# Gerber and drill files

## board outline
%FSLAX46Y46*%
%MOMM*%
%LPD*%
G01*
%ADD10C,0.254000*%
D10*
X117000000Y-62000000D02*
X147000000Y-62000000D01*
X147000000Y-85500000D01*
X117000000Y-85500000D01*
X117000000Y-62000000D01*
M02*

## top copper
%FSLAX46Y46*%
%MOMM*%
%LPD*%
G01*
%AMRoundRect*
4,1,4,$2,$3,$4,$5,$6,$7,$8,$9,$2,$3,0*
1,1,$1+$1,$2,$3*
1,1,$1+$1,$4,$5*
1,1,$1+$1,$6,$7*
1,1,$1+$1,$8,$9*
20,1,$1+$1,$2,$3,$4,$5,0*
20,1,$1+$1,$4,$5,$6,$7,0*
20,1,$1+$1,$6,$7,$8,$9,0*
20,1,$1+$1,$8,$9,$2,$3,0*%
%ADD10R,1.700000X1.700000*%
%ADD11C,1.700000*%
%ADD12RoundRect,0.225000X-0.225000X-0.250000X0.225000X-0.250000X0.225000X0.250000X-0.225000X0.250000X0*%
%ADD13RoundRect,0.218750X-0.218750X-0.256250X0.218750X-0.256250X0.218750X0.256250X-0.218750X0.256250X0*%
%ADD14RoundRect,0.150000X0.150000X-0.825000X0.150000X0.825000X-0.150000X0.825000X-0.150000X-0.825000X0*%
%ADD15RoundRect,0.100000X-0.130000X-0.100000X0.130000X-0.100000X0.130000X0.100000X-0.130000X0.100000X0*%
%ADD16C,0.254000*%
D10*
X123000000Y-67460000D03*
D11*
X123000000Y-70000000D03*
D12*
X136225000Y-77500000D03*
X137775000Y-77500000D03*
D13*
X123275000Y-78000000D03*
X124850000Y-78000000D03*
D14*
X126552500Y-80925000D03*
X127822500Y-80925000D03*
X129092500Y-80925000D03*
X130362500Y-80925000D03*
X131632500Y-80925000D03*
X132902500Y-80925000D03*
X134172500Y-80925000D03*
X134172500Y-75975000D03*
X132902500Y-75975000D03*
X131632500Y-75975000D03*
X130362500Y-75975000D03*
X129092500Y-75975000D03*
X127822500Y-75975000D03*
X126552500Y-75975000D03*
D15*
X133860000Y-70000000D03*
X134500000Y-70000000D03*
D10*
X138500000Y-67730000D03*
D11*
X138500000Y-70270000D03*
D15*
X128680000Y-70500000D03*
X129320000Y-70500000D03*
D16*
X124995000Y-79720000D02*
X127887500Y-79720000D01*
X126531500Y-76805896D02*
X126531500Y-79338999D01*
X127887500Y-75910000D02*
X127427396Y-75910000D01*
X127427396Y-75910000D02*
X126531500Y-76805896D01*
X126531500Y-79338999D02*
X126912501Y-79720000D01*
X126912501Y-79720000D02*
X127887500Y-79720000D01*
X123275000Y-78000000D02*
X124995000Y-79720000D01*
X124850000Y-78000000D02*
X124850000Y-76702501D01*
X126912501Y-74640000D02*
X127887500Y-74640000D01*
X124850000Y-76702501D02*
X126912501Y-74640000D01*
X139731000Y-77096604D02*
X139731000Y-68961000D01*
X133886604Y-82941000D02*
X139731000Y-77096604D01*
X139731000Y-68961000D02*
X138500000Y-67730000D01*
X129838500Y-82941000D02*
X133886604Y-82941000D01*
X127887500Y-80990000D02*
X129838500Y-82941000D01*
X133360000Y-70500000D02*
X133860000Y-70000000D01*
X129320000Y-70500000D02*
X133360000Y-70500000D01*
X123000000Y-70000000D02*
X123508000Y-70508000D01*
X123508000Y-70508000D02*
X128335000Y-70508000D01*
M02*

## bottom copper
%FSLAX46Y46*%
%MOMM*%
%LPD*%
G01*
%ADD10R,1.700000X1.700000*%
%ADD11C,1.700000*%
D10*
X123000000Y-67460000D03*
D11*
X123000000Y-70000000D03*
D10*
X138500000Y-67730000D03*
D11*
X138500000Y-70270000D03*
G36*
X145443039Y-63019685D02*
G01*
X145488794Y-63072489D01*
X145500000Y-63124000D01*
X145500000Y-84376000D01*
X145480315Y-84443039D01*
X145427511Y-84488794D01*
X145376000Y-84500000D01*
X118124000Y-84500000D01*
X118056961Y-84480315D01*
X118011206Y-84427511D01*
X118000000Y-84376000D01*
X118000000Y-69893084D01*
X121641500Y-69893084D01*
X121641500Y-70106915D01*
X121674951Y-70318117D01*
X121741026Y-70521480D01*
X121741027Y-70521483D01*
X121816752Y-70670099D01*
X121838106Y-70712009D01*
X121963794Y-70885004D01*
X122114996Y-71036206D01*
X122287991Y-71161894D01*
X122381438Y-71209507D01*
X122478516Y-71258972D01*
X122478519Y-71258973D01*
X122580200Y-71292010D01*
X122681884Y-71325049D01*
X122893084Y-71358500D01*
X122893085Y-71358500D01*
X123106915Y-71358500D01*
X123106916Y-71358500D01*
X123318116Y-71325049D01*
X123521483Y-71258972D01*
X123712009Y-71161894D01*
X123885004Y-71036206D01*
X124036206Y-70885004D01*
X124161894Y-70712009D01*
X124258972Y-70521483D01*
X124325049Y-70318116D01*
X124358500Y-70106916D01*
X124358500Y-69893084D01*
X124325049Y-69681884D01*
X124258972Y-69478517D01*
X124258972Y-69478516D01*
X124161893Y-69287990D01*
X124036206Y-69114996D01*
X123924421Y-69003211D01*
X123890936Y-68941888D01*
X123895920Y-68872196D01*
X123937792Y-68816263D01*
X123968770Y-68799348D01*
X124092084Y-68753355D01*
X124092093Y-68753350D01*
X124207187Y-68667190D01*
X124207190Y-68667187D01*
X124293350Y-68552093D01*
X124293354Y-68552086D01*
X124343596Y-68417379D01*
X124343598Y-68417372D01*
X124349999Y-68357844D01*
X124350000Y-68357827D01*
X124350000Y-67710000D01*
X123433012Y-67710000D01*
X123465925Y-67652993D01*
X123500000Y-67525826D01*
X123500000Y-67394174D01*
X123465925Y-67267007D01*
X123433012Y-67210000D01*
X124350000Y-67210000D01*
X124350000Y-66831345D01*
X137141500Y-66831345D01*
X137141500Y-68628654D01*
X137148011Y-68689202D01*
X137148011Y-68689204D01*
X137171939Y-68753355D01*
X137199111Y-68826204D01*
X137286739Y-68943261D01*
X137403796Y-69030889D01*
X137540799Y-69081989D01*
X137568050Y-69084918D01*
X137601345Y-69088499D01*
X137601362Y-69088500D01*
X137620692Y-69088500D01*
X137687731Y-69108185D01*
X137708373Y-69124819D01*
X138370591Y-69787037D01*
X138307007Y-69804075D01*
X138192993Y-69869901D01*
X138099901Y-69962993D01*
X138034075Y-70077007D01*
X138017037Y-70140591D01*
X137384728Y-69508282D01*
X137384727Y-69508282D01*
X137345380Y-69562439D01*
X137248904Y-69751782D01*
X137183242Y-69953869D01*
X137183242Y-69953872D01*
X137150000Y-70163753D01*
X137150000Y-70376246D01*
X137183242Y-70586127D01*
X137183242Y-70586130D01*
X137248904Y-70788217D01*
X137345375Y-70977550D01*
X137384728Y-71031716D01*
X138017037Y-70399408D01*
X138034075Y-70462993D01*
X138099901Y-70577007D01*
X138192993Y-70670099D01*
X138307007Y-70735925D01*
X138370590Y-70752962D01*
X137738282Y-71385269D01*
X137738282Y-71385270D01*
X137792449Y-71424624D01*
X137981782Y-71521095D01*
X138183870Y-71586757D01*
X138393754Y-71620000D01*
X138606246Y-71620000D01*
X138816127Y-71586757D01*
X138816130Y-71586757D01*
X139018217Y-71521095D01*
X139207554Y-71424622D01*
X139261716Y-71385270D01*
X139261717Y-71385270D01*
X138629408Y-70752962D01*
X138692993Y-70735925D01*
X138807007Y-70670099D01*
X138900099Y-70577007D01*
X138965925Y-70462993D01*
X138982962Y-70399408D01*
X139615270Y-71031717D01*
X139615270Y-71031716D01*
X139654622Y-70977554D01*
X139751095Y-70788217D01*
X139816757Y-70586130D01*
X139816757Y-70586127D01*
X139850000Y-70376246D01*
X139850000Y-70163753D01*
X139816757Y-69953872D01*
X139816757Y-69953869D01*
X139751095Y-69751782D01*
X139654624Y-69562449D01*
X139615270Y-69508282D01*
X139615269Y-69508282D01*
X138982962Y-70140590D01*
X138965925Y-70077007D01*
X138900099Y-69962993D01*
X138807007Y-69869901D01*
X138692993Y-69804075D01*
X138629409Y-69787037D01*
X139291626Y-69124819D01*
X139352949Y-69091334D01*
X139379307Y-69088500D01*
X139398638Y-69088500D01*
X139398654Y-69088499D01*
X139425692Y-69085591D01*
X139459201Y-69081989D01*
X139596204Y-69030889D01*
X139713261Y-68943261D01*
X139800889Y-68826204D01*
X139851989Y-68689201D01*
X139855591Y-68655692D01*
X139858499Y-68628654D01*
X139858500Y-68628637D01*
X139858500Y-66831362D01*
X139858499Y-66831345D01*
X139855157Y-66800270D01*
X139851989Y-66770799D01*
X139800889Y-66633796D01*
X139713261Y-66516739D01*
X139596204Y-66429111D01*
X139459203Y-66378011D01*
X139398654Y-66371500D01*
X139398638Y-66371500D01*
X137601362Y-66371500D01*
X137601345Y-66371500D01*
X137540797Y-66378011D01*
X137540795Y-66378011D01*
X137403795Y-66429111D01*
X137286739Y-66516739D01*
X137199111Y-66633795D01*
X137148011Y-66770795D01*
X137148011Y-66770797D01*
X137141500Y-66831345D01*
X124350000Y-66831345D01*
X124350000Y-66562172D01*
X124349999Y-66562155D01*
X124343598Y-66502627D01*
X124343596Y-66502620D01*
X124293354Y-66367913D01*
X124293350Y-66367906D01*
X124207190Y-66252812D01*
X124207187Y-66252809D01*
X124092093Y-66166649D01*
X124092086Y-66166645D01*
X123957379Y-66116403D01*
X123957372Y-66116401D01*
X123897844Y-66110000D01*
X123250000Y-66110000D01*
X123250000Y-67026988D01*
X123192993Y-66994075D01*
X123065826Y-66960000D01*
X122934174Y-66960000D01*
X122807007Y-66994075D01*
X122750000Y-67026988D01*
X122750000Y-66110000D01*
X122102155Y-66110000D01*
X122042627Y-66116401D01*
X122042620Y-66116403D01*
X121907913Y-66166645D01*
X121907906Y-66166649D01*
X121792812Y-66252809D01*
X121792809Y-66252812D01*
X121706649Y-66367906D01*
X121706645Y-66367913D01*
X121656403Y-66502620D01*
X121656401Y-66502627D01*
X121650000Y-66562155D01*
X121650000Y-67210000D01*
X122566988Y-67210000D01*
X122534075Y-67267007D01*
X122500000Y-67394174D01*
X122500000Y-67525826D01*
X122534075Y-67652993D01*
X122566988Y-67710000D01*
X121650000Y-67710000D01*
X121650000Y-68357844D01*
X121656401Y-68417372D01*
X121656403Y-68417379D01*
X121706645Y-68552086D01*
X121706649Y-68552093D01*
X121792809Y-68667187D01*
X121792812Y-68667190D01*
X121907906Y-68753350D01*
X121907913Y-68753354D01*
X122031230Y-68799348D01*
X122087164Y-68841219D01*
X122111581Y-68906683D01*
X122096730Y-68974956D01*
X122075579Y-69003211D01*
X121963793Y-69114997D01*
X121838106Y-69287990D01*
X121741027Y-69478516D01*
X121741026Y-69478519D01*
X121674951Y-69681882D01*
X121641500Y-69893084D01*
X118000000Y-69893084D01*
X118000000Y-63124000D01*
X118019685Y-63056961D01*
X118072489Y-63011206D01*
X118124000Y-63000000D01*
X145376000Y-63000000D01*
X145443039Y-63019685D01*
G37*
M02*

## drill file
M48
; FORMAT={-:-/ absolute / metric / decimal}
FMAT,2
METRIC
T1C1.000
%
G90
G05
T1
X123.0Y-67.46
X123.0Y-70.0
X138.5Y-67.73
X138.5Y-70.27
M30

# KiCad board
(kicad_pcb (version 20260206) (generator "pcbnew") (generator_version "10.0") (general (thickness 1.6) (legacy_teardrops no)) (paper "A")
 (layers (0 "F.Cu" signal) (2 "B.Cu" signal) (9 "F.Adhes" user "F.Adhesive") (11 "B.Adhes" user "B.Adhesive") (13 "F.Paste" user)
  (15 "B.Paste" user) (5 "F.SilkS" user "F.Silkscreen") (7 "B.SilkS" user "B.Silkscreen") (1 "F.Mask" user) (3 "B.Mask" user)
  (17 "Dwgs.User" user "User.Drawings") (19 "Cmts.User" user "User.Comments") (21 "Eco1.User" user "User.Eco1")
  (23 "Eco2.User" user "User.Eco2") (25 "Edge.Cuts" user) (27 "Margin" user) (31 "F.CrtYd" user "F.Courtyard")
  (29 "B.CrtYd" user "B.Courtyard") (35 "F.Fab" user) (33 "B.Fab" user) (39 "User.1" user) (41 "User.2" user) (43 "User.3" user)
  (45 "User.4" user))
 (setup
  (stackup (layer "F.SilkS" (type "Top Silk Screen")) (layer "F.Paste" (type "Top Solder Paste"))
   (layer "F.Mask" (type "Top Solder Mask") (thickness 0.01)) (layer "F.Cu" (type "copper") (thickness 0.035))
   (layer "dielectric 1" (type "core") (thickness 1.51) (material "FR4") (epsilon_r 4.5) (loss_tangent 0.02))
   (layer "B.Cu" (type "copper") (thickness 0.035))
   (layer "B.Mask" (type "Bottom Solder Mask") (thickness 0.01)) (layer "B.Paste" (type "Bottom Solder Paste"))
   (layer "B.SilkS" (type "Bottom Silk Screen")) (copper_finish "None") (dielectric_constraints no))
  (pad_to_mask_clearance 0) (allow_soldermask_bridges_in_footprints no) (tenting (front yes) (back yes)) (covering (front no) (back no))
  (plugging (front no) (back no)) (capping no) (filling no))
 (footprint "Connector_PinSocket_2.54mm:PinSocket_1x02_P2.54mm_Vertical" (layer "F.Cu") (at 123 67.46)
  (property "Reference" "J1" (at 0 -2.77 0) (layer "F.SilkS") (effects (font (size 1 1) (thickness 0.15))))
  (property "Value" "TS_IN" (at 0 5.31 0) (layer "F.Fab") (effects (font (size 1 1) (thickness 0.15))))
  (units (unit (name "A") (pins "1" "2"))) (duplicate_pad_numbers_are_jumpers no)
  (pad "1" thru_hole rect (at 0 0) (size 1.7 1.7) (drill 1) (layers "*.Cu" "*.Mask") (remove_unused_layers no) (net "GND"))
  (pad "2" thru_hole circle (at 0 2.54) (size 1.7 1.7) (drill 1) (layers "*.Cu" "*.Mask") (remove_unused_layers no) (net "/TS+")))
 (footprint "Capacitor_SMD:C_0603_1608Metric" (layer "F.Cu") (at 137 77.5)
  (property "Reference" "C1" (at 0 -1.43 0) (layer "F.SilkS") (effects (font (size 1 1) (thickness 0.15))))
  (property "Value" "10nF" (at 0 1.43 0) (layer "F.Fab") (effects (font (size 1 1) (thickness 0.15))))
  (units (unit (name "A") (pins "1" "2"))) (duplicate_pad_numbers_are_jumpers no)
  (pad "1" smd roundrect (at -0.775 0) (size 0.9 0.95) (layers "F.Cu" "F.Mask" "F.Paste") (roundrect_rratio 0.25) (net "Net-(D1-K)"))
  (pad "2" smd roundrect (at 0.775 0) (size 0.9 0.95) (layers "F.Cu" "F.Mask" "F.Paste") (roundrect_rratio 0.25) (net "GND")))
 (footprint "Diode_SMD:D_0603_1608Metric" (layer "F.Cu") (at 124.0625 78)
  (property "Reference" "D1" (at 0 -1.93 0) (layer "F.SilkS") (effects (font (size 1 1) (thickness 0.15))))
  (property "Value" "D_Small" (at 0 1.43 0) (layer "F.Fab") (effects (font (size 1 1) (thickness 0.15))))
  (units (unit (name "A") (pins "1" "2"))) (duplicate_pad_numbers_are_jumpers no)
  (pad "1" smd roundrect (at -0.7875 0) (size 0.875 0.95) (layers "F.Cu" "F.Mask" "F.Paste") (roundrect_rratio 0.25) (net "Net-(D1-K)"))
  (pad "2" smd roundrect (at 0.7875 0) (size 0.875 0.95) (layers "F.Cu" "F.Mask" "F.Paste") (roundrect_rratio 0.25) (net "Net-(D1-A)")))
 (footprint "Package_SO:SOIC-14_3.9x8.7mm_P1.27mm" (layer "F.Cu") (at 130.3625 78.45 90)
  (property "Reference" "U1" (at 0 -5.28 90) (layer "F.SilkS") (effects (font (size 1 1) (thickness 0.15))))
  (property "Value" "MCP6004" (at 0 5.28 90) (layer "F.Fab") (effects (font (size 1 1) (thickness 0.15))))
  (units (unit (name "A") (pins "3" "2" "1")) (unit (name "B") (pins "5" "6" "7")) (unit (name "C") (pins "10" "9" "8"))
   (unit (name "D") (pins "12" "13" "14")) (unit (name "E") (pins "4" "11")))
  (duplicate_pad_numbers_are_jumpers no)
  (pad "1" smd roundrect (at -2.475 -3.81 90) (size 1.95 0.6) (layers "F.Cu" "F.Mask" "F.Paste") (roundrect_rratio 0.25) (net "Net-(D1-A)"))
  (pad "2" smd roundrect (at -2.475 -2.54 90) (size 1.95 0.6) (layers "F.Cu" "F.Mask" "F.Paste") (roundrect_rratio 0.25) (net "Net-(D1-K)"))
  (pad "3" smd roundrect (at -2.475 -1.27 90) (size 1.95 0.6) (layers "F.Cu" "F.Mask" "F.Paste") (roundrect_rratio 0.25) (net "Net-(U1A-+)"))
  (pad "4" smd roundrect (at -2.475 0 90) (size 1.95 0.6) (layers "F.Cu" "F.Mask" "F.Paste") (roundrect_rratio 0.25))
  (pad "5" smd roundrect (at -2.475 1.27 90) (size 1.95 0.6) (layers "F.Cu" "F.Mask" "F.Paste") (roundrect_rratio 0.25) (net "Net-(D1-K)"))
  (pad "6" smd roundrect (at -2.475 2.54 90) (size 1.95 0.6) (layers "F.Cu" "F.Mask" "F.Paste") (roundrect_rratio 0.25) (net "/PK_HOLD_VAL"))
  (pad "7" smd roundrect (at -2.475 3.81 90) (size 1.95 0.6) (layers "F.Cu" "F.Mask" "F.Paste") (roundrect_rratio 0.25) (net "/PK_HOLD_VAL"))
  (pad "8" smd roundrect (at 2.475 3.81 90) (size 1.95 0.6) (layers "F.Cu" "F.Mask" "F.Paste") (roundrect_rratio 0.25)
   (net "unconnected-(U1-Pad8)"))
  (pad "9" smd roundrect (at 2.475 2.54 90) (size 1.95 0.6) (layers "F.Cu" "F.Mask" "F.Paste") (roundrect_rratio 0.25)
   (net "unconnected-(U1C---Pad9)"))
  (pad "10" smd roundrect (at 2.475 1.27 90) (size 1.95 0.6) (layers "F.Cu" "F.Mask" "F.Paste") (roundrect_rratio 0.25)
   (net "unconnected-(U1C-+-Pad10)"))
  (pad "11" smd roundrect (at 2.475 0 90) (size 1.95 0.6) (layers "F.Cu" "F.Mask" "F.Paste") (roundrect_rratio 0.25))
  (pad "12" smd roundrect (at 2.475 -1.27 90) (size 1.95 0.6) (layers "F.Cu" "F.Mask" "F.Paste") (roundrect_rratio 0.25))
  (pad "13" smd roundrect (at 2.475 -2.54 90) (size 1.95 0.6) (layers "F.Cu" "F.Mask" "F.Paste") (roundrect_rratio 0.25))
  (pad "14" smd roundrect (at 2.475 -3.81 90) (size 1.95 0.6) (layers "F.Cu" "F.Mask" "F.Paste") (roundrect_rratio 0.25)))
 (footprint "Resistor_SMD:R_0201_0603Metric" (layer "F.Cu") (at 134.18 70)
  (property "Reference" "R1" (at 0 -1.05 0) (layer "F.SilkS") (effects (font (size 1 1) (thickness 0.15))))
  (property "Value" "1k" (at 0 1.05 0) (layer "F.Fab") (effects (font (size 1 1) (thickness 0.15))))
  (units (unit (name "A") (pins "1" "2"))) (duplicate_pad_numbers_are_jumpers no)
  (pad "" smd roundrect (at -0.345 0) (size 0.318 0.36) (layers "F.Paste") (roundrect_rratio 0.25))
  (pad "" smd roundrect (at 0.345 0) (size 0.318 0.36) (layers "F.Paste") (roundrect_rratio 0.25))
  (pad "1" smd roundrect (at -0.32 0) (size 0.46 0.4) (layers "F.Cu" "F.Mask") (roundrect_rratio 0.25) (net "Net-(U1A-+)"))
  (pad "2" smd roundrect (at 0.32 0) (size 0.46 0.4) (layers "F.Cu" "F.Mask") (roundrect_rratio 0.25) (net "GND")))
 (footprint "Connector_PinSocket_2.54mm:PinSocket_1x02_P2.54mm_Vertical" (layer "F.Cu") (at 138.5 67.73)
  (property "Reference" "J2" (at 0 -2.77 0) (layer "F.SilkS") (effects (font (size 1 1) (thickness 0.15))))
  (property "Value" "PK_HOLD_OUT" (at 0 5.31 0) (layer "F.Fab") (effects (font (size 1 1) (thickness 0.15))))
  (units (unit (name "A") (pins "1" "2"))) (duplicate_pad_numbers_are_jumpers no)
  (pad "1" thru_hole rect (at 0 0) (size 1.7 1.7) (drill 1) (layers "*.Cu" "*.Mask") (remove_unused_layers no) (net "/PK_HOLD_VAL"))
  (pad "2" thru_hole circle (at 0 2.54) (size 1.7 1.7) (drill 1) (layers "*.Cu" "*.Mask") (remove_unused_layers no) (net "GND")))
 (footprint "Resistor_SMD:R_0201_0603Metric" (layer "F.Cu") (at 129 70.5)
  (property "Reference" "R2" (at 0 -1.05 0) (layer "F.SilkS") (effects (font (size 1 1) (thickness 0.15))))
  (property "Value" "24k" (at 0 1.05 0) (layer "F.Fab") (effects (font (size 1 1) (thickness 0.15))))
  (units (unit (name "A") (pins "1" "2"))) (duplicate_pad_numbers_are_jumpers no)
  (pad "" smd roundrect (at -0.345 0) (size 0.318 0.36) (layers "F.Paste") (roundrect_rratio 0.25))
  (pad "" smd roundrect (at 0.345 0) (size 0.318 0.36) (layers "F.Paste") (roundrect_rratio 0.25))
  (pad "1" smd roundrect (at -0.32 0) (size 0.46 0.4) (layers "F.Cu" "F.Mask") (roundrect_rratio 0.25) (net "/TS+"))
  (pad "2" smd roundrect (at 0.32 0) (size 0.46 0.4) (layers "F.Cu" "F.Mask") (roundrect_rratio 0.25) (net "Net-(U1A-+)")))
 (gr_rect (start 117 62) (end 147 85.5) (stroke (width 0.254) (type solid)) (fill no) (layer "Edge.Cuts"))
 (segment (start 124.995 79.72) (end 127.8875 79.72) (width 0.254) (layer "F.Cu") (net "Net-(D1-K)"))
 (segment (start 126.5315 76.805896) (end 126.5315 79.338999) (width 0.254) (layer "F.Cu") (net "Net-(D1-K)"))
 (segment (start 127.8875 75.91) (end 127.427396 75.91) (width 0.254) (layer "F.Cu") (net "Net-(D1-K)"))
 (segment (start 127.427396 75.91) (end 126.5315 76.805896) (width 0.254) (layer "F.Cu") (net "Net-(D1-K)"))
 (segment (start 126.5315 79.338999) (end 126.912501 79.72) (width 0.254) (layer "F.Cu") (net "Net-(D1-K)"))
 (segment (start 126.912501 79.72) (end 127.8875 79.72) (width 0.254) (layer "F.Cu") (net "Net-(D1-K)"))
 (segment (start 123.275 78) (end 124.995 79.72) (width 0.254) (layer "F.Cu") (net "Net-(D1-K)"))
 (segment (start 124.85 78) (end 124.85 76.702501) (width 0.254) (layer "F.Cu") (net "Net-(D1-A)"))
 (segment (start 126.912501 74.64) (end 127.8875 74.64) (width 0.254) (layer "F.Cu") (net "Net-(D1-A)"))
 (segment (start 124.85 76.702501) (end 126.912501 74.64) (width 0.254) (layer "F.Cu") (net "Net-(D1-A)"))
 (segment (start 139.731 77.096604) (end 139.731 68.961) (width 0.254) (layer "F.Cu") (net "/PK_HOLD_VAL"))
 (segment (start 133.886604 82.941) (end 139.731 77.096604) (width 0.254) (layer "F.Cu") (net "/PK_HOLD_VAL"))
 (segment (start 139.731 68.961) (end 138.5 67.73) (width 0.254) (layer "F.Cu") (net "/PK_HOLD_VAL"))
 (segment (start 129.8385 82.941) (end 133.886604 82.941) (width 0.254) (layer "F.Cu") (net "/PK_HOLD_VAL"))
 (segment (start 127.8875 80.99) (end 129.8385 82.941) (width 0.254) (layer "F.Cu") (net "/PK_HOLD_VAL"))
 (segment (start 133.36 70.5) (end 133.86 70) (width 0.254) (layer "F.Cu") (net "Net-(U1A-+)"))
 (segment (start 129.32 70.5) (end 133.36 70.5) (width 0.254) (layer "F.Cu") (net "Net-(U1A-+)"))
 (segment (start 123 70) (end 123.508 70.508) (width 0.254) (layer "F.Cu") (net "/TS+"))
 (segment (start 123.508 70.508) (end 128.335 70.508) (width 0.254) (layer "F.Cu") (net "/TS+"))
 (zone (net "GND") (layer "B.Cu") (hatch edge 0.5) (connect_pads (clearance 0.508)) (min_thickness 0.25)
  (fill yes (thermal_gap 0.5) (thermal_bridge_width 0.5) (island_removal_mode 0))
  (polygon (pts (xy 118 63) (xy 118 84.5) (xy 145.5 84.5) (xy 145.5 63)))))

